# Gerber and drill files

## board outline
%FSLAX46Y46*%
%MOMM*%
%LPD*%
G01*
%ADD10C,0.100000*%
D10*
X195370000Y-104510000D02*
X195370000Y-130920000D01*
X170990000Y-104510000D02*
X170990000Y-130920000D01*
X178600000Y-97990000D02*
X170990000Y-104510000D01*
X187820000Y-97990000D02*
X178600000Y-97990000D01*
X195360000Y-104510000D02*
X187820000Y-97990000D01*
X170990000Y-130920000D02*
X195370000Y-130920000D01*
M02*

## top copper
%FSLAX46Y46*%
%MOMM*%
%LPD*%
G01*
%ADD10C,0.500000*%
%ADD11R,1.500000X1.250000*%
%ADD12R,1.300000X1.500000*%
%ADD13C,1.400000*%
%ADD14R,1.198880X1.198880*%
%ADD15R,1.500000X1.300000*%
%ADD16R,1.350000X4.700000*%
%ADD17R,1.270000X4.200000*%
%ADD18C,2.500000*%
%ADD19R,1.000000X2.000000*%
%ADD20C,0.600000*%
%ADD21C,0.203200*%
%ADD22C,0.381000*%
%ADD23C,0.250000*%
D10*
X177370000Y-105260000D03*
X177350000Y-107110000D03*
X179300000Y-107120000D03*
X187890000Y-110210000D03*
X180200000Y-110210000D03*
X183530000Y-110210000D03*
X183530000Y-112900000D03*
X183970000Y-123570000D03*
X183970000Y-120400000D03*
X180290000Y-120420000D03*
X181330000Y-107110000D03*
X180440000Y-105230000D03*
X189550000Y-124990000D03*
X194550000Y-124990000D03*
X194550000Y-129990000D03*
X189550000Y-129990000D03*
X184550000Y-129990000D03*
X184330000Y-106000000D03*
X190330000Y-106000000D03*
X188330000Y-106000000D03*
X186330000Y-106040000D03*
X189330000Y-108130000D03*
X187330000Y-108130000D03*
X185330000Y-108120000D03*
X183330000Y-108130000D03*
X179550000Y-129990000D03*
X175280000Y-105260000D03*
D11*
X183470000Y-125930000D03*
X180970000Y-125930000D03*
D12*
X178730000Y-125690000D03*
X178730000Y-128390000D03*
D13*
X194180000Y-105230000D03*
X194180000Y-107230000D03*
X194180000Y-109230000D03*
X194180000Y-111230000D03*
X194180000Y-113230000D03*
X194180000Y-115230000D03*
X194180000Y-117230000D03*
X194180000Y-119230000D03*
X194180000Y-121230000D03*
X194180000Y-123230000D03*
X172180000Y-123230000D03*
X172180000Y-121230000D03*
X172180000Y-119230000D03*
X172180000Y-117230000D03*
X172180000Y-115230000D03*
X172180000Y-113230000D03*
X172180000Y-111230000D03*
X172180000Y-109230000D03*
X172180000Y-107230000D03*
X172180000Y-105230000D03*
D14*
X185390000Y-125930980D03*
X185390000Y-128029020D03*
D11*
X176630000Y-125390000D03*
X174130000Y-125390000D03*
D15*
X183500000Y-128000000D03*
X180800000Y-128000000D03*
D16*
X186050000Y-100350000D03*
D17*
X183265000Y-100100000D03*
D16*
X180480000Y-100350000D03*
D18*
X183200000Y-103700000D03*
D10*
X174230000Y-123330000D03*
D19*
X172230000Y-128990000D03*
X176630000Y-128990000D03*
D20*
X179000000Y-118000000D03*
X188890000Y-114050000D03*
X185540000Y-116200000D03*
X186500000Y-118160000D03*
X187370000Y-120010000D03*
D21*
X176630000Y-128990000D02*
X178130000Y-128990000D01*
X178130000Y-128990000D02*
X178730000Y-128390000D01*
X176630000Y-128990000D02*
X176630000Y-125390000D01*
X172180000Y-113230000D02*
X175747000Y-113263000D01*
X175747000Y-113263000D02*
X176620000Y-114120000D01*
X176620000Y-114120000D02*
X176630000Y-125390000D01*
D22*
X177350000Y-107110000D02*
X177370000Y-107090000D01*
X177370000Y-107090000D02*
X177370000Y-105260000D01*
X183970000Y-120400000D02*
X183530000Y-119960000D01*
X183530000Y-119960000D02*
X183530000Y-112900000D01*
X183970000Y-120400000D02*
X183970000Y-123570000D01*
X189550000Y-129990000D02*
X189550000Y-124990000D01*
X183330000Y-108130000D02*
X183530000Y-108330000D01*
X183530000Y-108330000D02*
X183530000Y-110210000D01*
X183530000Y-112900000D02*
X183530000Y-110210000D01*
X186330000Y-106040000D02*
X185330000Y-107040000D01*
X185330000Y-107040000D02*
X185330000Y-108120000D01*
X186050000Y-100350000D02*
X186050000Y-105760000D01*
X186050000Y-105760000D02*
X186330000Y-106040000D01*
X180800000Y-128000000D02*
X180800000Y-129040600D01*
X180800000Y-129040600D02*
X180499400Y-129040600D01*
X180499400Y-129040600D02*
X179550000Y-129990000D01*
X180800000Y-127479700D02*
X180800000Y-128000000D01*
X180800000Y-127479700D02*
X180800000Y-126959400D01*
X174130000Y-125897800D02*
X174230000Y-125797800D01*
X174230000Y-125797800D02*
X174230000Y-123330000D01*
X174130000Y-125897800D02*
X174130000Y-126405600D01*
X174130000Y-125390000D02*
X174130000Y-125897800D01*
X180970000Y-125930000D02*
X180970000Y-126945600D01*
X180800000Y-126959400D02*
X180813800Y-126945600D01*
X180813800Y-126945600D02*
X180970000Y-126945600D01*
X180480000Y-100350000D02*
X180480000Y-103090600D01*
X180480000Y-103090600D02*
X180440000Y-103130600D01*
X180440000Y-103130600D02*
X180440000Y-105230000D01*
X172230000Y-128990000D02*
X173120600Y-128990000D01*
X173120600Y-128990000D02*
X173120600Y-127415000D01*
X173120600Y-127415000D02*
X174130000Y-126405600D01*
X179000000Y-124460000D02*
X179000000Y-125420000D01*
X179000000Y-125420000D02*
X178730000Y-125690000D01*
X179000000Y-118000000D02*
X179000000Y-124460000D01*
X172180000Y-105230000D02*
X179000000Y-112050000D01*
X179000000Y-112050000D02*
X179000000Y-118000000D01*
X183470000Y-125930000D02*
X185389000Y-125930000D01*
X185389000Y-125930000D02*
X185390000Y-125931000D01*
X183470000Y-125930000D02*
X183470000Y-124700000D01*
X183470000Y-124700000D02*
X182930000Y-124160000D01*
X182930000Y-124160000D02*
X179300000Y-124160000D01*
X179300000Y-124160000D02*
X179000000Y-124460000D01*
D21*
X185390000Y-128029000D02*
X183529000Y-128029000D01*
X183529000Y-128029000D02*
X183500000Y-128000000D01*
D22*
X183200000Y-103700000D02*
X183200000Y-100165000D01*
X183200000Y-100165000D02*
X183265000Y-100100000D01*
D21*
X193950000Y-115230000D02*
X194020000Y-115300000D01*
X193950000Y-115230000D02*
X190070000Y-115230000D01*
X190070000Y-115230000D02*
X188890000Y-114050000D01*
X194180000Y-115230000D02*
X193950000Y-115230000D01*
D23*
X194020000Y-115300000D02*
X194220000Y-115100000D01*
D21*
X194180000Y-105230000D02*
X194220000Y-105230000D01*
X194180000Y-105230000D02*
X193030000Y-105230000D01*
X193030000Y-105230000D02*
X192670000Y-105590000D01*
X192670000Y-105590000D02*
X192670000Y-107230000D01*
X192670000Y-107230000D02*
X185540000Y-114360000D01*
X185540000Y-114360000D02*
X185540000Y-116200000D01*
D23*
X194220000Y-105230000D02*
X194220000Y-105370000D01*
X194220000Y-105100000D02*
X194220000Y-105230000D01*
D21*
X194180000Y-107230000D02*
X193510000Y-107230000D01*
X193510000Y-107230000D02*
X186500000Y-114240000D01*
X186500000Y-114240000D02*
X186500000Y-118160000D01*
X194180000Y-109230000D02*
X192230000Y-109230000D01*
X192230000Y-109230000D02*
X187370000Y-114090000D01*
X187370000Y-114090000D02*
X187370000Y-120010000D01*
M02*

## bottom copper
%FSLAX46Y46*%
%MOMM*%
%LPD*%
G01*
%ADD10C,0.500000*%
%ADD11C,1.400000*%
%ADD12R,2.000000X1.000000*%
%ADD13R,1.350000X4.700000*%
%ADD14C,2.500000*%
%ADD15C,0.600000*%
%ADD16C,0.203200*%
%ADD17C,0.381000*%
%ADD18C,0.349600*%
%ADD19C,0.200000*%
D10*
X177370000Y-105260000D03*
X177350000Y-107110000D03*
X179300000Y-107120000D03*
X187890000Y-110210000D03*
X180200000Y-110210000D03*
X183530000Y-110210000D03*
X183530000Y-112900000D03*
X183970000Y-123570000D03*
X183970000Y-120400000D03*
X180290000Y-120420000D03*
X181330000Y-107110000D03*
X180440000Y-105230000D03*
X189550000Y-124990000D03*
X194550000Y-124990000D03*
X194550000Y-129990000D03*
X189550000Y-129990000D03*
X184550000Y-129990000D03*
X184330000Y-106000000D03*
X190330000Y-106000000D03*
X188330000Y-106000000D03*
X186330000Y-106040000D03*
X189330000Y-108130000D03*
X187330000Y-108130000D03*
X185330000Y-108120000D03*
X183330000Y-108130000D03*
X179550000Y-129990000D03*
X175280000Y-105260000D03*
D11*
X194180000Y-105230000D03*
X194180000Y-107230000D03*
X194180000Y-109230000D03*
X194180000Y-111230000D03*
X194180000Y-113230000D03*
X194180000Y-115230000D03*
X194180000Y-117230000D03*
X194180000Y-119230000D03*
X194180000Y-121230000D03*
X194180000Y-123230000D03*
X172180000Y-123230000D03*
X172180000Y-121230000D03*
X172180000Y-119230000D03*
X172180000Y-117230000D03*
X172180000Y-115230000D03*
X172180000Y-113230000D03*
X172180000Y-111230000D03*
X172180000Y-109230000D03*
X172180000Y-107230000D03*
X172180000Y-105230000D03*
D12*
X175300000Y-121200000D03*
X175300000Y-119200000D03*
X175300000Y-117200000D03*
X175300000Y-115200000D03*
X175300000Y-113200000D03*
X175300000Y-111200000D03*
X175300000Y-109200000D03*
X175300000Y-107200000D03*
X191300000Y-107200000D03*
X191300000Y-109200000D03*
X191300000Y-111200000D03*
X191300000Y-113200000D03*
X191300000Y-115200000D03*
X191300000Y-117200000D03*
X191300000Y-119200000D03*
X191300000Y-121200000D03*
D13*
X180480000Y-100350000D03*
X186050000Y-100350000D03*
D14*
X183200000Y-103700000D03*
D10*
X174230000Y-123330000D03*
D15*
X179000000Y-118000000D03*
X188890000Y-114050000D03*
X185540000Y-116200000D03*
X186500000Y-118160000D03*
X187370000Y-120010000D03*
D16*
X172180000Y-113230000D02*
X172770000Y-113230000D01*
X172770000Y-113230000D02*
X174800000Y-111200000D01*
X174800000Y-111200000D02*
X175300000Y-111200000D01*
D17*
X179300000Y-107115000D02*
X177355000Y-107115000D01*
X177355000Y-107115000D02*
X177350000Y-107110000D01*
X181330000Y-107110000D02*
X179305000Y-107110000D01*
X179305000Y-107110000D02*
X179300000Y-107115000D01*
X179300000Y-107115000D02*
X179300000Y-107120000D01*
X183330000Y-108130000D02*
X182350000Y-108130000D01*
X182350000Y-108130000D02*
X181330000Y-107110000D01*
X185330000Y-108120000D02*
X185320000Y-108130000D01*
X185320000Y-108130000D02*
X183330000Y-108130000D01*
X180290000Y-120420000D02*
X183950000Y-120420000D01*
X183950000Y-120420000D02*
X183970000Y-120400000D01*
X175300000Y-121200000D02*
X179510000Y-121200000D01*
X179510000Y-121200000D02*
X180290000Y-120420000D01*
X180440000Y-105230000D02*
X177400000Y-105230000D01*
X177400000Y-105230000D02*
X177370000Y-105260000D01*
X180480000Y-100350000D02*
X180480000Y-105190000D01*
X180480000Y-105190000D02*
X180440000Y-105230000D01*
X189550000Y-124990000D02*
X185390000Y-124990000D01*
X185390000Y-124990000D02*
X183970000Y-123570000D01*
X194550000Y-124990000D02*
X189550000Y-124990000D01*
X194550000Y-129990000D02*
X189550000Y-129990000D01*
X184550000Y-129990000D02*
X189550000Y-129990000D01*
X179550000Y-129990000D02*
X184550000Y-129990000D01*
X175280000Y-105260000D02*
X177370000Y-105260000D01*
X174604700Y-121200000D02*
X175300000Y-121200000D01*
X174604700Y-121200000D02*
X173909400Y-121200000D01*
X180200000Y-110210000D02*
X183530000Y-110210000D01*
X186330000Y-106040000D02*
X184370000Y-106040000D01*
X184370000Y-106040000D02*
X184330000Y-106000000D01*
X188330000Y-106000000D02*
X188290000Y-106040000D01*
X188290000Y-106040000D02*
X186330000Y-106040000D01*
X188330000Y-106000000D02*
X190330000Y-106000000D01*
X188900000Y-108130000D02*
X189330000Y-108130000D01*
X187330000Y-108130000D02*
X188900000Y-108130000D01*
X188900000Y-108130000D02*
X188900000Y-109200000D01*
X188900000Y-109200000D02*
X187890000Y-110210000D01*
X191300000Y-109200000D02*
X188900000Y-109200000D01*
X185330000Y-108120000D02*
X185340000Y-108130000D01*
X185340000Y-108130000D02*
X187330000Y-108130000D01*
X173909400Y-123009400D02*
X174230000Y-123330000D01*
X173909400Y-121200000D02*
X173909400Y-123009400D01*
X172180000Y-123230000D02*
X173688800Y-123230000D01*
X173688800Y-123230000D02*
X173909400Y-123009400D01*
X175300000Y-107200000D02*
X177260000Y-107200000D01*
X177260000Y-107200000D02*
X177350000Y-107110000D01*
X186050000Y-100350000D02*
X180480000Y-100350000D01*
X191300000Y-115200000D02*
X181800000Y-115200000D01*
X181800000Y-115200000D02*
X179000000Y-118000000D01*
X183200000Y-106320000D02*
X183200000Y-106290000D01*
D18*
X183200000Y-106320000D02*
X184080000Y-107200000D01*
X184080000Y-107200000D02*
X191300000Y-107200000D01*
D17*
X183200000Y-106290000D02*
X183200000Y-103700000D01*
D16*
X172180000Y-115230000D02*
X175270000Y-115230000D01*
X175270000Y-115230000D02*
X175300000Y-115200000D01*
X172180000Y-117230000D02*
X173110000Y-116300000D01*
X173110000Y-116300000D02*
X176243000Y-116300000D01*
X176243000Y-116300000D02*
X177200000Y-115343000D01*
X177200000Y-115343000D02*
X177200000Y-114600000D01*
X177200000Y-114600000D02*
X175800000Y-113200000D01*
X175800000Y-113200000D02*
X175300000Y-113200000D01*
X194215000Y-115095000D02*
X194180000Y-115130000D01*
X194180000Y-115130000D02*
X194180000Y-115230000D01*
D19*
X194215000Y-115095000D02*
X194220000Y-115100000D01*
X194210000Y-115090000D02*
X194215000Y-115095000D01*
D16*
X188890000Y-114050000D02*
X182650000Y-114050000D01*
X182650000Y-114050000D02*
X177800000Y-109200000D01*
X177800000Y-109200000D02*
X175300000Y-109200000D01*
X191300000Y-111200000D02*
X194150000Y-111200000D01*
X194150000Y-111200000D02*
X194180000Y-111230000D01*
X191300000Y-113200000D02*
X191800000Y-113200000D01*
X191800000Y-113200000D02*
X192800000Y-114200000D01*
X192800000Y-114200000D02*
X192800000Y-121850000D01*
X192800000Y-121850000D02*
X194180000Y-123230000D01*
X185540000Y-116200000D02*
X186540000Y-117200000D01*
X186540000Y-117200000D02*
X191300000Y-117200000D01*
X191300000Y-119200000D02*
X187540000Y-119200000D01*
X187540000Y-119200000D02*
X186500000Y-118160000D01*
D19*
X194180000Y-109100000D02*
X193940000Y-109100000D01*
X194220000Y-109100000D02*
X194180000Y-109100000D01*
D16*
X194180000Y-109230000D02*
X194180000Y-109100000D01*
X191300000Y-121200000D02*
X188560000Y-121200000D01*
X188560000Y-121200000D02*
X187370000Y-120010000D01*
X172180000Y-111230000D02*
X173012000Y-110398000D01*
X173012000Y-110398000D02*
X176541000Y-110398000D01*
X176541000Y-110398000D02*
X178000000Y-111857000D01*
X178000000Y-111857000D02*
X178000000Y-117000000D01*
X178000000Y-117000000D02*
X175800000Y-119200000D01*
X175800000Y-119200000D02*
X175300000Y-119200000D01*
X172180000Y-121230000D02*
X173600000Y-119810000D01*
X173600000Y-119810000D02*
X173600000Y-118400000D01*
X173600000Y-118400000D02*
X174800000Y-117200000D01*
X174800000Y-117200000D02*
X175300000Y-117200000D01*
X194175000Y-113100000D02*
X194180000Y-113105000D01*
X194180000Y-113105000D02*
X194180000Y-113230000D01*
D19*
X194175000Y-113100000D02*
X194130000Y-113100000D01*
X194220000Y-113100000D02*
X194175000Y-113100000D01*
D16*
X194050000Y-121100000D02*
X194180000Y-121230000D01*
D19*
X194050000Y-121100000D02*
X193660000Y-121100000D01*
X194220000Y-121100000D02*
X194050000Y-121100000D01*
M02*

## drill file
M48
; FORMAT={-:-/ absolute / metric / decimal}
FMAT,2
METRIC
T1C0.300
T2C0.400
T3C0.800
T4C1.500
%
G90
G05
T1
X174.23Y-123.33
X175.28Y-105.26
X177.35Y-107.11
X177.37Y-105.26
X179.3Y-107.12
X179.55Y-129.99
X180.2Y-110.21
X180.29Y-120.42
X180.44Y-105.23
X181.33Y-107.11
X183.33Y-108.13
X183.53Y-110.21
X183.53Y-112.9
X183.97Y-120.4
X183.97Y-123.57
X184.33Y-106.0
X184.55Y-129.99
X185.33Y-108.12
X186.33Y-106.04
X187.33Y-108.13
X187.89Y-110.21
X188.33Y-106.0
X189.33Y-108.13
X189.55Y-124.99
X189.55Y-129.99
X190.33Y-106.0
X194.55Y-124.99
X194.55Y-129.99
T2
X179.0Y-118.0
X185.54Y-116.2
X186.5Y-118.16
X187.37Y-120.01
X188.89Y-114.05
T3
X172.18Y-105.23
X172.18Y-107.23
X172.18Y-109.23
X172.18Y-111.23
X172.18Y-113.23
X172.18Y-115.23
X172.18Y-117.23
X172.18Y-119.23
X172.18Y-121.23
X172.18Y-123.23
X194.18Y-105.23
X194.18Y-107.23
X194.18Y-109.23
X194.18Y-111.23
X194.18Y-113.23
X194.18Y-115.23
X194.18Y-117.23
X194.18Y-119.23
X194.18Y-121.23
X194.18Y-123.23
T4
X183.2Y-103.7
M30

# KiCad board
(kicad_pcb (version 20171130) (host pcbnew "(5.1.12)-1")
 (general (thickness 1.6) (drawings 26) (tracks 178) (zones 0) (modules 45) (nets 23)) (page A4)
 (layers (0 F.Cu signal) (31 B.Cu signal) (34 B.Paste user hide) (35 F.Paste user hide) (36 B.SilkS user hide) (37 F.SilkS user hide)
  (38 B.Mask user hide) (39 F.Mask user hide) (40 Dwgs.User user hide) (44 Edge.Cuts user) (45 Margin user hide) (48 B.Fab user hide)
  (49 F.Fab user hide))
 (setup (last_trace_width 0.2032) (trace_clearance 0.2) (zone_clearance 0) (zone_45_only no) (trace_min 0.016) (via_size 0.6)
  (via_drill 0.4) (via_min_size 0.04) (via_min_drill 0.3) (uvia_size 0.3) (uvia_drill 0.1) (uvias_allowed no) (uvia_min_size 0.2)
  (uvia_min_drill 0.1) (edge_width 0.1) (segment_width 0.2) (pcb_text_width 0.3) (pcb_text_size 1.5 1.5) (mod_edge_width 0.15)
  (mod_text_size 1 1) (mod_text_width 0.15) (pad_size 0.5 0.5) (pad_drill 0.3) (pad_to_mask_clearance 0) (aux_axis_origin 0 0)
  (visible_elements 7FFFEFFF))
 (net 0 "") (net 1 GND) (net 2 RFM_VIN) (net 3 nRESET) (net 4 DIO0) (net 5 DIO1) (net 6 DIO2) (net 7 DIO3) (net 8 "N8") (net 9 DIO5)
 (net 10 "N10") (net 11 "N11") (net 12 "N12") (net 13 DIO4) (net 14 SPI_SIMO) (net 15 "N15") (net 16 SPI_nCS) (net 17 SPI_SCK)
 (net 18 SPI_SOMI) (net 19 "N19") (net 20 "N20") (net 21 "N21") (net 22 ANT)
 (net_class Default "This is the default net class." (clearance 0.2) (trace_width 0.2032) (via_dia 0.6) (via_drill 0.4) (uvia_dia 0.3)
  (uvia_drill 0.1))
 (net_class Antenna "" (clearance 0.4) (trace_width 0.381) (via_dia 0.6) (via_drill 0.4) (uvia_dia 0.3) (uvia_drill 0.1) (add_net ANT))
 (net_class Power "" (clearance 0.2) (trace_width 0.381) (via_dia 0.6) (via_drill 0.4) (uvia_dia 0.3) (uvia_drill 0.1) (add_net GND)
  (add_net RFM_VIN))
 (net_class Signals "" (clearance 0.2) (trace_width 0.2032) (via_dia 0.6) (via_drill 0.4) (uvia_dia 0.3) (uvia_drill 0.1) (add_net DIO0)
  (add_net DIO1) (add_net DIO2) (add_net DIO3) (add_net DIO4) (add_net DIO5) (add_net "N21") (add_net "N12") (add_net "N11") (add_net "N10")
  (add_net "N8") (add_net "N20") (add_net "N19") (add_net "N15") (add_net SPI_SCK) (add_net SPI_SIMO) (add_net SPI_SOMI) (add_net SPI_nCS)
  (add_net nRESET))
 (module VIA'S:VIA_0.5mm (layer F.Cu) (at 177.37 105.26)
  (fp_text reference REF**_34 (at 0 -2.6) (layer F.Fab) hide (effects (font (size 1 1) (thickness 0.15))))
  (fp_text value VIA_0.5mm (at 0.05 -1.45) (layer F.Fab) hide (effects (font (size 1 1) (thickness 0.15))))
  (pad 1 thru_hole circle (at 0 0) (size 0.5 0.5) (drill 0.3) (layers *.Cu) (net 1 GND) (zone_connect 2)))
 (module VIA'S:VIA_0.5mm (layer F.Cu) (at 177.35 107.11)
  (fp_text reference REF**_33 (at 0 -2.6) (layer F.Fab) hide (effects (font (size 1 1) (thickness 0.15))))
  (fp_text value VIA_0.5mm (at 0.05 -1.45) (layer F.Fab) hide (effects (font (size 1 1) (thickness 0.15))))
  (pad 1 thru_hole circle (at 0 0) (size 0.5 0.5) (drill 0.3) (layers *.Cu) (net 1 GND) (zone_connect 2)))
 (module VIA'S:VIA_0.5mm (layer F.Cu) (at 179.3 107.12)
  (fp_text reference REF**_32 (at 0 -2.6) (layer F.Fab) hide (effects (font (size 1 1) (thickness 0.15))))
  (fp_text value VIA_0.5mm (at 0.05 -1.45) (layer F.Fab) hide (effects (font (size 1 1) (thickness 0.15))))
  (pad 1 thru_hole circle (at 0 0) (size 0.5 0.5) (drill 0.3) (layers *.Cu) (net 1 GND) (zone_connect 2)))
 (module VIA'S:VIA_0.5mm (layer F.Cu) (at 186.03 105.9)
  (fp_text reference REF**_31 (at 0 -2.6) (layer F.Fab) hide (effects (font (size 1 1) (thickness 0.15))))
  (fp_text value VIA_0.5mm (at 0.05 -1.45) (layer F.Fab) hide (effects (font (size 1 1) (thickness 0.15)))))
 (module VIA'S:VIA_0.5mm (layer F.Cu) (at 187.89 110.29)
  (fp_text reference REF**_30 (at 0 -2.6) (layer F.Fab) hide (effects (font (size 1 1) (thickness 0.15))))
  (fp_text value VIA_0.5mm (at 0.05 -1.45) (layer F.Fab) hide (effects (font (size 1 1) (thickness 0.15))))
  (pad 1 thru_hole circle (at 0 -0.08) (size 0.5 0.5) (drill 0.3) (layers *.Cu) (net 1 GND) (zone_connect 2)))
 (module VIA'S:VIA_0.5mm (layer F.Cu) (at 180.2 110.23)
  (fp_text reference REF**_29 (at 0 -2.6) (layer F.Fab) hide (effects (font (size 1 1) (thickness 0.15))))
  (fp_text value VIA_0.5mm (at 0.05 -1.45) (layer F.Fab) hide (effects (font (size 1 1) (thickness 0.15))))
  (pad 1 thru_hole circle (at 0 -0.02) (size 0.5 0.5) (drill 0.3) (layers *.Cu) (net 1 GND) (zone_connect 2)))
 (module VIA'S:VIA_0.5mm (layer F.Cu) (at 183.53 110.21)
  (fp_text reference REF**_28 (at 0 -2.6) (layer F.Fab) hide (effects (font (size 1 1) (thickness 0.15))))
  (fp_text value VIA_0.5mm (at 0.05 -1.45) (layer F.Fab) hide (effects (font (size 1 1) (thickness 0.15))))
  (pad 1 thru_hole circle (at 0 0) (size 0.5 0.5) (drill 0.3) (layers *.Cu) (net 1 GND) (zone_connect 2)))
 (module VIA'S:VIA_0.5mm (layer F.Cu) (at 183.54 112.9)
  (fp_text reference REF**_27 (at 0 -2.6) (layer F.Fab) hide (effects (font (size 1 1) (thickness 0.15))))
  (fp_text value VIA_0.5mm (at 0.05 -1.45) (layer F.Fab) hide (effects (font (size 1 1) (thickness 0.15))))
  (pad 1 thru_hole circle (at -0.01 0) (size 0.5 0.5) (drill 0.3) (layers *.Cu) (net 1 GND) (zone_connect 2)))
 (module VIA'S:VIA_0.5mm (layer F.Cu) (at 183.97 123.57)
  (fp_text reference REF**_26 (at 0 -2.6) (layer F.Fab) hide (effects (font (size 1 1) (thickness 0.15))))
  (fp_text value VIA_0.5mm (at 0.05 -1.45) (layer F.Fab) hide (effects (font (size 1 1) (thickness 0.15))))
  (pad 1 thru_hole circle (at 0 0) (size 0.5 0.5) (drill 0.3) (layers *.Cu) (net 1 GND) (zone_connect 2)))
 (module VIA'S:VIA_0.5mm (layer F.Cu) (at 183.97 120.4)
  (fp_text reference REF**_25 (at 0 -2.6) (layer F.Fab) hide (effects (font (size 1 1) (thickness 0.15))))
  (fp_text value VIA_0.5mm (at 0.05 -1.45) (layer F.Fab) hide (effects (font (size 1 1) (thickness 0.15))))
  (pad 1 thru_hole circle (at 0 0) (size 0.5 0.5) (drill 0.3) (layers *.Cu) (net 1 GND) (zone_connect 2)))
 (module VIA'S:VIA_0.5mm (layer F.Cu) (at 180.29 120.42)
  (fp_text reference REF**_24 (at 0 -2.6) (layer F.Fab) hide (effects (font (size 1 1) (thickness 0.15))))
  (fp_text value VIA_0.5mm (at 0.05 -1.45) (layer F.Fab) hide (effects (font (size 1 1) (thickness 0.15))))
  (pad 1 thru_hole circle (at 0 0) (size 0.5 0.5) (drill 0.3) (layers *.Cu) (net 1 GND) (zone_connect 2)))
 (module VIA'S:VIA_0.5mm (layer F.Cu) (at 181.33 107.11)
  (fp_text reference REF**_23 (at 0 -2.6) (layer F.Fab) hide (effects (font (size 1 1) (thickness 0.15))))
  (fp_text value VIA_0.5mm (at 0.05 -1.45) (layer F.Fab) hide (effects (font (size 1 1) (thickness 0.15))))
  (pad 1 thru_hole circle (at 0 0) (size 0.5 0.5) (drill 0.3) (layers *.Cu) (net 1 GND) (zone_connect 2)))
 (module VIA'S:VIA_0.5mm (layer F.Cu) (at 180.44 105.23)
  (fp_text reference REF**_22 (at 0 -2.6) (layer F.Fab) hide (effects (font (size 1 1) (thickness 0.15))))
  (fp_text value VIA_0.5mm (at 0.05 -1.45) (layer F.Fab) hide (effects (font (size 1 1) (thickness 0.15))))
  (pad 1 thru_hole circle (at 0 0) (size 0.5 0.5) (drill 0.3) (layers *.Cu) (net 1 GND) (zone_connect 2)))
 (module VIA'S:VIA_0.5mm (layer F.Cu) (at 189.55 124.99)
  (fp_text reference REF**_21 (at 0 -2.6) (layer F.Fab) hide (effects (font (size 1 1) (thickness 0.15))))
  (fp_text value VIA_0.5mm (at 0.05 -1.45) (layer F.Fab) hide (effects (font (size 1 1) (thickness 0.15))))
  (pad 1 thru_hole circle (at 0 0) (size 0.5 0.5) (drill 0.3) (layers *.Cu) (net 1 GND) (zone_connect 2)))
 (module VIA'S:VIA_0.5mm (layer F.Cu) (at 194.55 124.99)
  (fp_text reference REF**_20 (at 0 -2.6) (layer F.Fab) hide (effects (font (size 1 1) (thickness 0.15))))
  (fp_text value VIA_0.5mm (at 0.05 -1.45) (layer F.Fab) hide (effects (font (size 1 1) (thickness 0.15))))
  (pad 1 thru_hole circle (at 0 0) (size 0.5 0.5) (drill 0.3) (layers *.Cu) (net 1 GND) (zone_connect 2)))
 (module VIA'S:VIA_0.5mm (layer F.Cu) (at 194.55 129.99)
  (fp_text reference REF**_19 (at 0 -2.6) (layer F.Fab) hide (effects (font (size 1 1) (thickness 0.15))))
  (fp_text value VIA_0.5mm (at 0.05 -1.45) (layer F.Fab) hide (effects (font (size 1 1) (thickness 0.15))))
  (pad 1 thru_hole circle (at 0 0) (size 0.5 0.5) (drill 0.3) (layers *.Cu) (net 1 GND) (zone_connect 2)))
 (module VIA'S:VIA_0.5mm (layer F.Cu) (at 189.55 129.99)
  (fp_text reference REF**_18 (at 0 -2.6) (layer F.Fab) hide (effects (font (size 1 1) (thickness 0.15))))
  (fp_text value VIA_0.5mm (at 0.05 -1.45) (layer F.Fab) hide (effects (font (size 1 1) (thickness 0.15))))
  (pad 1 thru_hole circle (at 0 0) (size 0.5 0.5) (drill 0.3) (layers *.Cu) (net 1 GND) (zone_connect 2)))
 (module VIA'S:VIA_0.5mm (layer F.Cu) (at 184.55 129.99)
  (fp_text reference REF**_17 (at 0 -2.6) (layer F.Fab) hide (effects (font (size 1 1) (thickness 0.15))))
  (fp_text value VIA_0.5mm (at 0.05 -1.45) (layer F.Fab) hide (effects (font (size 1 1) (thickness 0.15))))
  (pad 1 thru_hole circle (at 0 0) (size 0.5 0.5) (drill 0.3) (layers *.Cu) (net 1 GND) (zone_connect 2)))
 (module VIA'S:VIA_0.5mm (layer F.Cu) (at 184.33 106.67)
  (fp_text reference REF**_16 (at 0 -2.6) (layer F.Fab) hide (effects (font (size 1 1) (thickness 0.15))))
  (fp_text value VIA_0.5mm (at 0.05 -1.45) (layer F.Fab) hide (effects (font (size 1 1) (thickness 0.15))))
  (pad 1 thru_hole circle (at 0 -0.67) (size 0.5 0.5) (drill 0.3) (layers *.Cu) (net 1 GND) (zone_connect 2)))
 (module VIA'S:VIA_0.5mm (layer F.Cu) (at 189.33 106.67)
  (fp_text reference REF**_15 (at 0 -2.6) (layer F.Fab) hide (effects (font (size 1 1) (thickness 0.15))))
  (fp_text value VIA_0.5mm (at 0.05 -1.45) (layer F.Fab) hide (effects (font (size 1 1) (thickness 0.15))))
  (pad 1 thru_hole circle (at 1 -0.67) (size 0.5 0.5) (drill 0.3) (layers *.Cu) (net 1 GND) (zone_connect 2)))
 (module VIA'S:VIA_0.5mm (layer F.Cu) (at 188.33 106.67)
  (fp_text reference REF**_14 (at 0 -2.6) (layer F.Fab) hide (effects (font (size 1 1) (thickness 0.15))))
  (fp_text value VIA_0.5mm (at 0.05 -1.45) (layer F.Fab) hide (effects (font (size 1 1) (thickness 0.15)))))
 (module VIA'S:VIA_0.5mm (layer F.Cu) (at 187.33 106.67)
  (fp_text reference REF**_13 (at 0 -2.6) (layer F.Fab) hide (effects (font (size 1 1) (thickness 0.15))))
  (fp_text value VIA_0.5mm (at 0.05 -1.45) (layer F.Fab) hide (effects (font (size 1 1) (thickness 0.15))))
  (pad 1 thru_hole circle (at 1 -0.67) (size 0.5 0.5) (drill 0.3) (layers *.Cu) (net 1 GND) (zone_connect 2)))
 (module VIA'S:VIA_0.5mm (layer F.Cu) (at 186.33 106.67)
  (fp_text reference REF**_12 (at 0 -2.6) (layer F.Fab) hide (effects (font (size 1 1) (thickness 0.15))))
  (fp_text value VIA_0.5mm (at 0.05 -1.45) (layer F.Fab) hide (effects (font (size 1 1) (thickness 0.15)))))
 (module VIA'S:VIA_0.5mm (layer F.Cu) (at 186.05 106.71)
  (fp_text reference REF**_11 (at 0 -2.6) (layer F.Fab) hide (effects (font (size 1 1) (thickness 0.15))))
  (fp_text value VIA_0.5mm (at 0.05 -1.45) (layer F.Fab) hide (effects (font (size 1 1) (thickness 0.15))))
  (pad 1 thru_hole circle (at 0.28 -0.67) (size 0.5 0.5) (drill 0.3) (layers *.Cu) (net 1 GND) (zone_connect 2)))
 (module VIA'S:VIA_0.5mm (layer F.Cu) (at 189.03 108.13)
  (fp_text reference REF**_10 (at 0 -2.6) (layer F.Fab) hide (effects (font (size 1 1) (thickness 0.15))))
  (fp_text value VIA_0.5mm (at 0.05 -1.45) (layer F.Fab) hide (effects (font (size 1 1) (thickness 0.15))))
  (pad 1 thru_hole circle (at 0.3 0) (size 0.5 0.5) (drill 0.3) (layers *.Cu) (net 1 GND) (zone_connect 2)))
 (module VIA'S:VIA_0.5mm (layer F.Cu) (at 188.03 108.13)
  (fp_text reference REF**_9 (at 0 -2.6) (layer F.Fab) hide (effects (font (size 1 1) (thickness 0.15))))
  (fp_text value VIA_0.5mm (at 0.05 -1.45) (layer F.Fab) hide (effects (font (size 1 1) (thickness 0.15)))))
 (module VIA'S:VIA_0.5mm (layer F.Cu) (at 187.03 108.13)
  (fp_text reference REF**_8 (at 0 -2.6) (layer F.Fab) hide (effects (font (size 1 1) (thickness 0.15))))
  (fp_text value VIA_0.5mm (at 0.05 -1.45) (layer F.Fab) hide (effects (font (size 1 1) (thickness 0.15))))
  (pad 1 thru_hole circle (at 0.3 0) (size 0.5 0.5) (drill 0.3) (layers *.Cu) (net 1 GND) (zone_connect 2)))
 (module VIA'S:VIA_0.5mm (layer F.Cu) (at 186.03 108.13)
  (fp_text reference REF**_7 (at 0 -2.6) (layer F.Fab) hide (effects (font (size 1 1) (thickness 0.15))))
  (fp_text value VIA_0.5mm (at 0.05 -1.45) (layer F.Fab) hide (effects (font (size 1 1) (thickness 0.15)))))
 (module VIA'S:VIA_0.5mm (layer F.Cu) (at 185.54 108.12)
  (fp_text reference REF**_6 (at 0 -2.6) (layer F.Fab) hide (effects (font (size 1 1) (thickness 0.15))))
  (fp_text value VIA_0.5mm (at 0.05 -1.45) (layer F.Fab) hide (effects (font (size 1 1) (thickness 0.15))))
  (pad 1 thru_hole circle (at -0.21 0) (size 0.5 0.5) (drill 0.3) (layers *.Cu) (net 1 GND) (zone_connect 2)))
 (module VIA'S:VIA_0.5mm (layer F.Cu) (at 184.03 108.13)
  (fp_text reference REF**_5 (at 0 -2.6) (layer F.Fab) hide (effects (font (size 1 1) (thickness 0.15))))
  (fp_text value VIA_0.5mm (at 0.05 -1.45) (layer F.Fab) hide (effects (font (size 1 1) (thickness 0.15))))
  (pad 1 thru_hole circle (at -0.7 0) (size 0.5 0.5) (drill 0.3) (layers *.Cu) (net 1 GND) (zone_connect 2)))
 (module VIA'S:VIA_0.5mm (layer F.Cu) (at 179.55 129.99)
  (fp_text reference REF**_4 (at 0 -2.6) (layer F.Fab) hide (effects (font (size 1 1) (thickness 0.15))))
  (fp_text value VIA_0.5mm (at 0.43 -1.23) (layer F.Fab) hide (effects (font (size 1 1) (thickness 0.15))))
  (pad 1 thru_hole circle (at 0 0) (size 0.5 0.5) (drill 0.3) (layers *.Cu) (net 1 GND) (zone_connect 2)))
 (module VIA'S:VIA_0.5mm (layer F.Cu) (at 175.28 105.26)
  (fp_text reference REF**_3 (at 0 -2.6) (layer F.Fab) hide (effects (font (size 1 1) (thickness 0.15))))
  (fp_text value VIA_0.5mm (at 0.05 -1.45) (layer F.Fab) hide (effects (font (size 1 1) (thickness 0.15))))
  (pad 1 thru_hole circle (at 0 0) (size 0.5 0.5) (drill 0.3) (layers *.Cu) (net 1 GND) (zone_connect 2)))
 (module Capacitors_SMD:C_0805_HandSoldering (layer F.Cu) (at 182.22 125.93 180)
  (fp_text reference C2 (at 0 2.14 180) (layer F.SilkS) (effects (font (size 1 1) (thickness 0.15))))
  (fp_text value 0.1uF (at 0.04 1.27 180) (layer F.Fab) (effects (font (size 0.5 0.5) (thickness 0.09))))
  (pad 1 smd rect (at -1.25 0 180) (size 1.5 1.25) (layers F.Cu F.Paste F.Mask) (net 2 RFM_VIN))
  (pad 2 smd rect (at 1.25 0 180) (size 1.5 1.25) (layers F.Cu F.Paste F.Mask) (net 1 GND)))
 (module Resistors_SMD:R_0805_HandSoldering (layer F.Cu) (at 178.73 127.04 270)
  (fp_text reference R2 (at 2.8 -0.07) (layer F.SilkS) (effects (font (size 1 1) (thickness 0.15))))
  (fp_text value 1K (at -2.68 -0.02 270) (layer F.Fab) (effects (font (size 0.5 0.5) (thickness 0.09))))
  (pad 1 smd rect (at -1.35 0 270) (size 1.5 1.3) (layers F.Cu F.Paste F.Mask) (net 2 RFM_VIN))
  (pad 2 smd rect (at 1.35 0 270) (size 1.5 1.3) (layers F.Cu F.Paste F.Mask) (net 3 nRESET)))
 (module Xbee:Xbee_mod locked (layer F.Cu) (at 172.18 105.23)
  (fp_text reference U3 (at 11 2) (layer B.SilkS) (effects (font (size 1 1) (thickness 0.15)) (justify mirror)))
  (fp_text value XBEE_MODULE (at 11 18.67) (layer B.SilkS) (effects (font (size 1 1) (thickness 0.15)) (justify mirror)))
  (pad 20 thru_hole circle (at 22 0) (size 1.4 1.4) (drill 0.8) (layers *.Cu *.Mask) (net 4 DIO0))
  (pad 19 thru_hole circle (at 22 2) (size 1.4 1.4) (drill 0.8) (layers *.Cu *.Mask) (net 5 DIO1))
  (pad 18 thru_hole circle (at 22 4) (size 1.4 1.4) (drill 0.8) (layers *.Cu *.Mask) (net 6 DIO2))
  (pad 17 thru_hole circle (at 22 6) (size 1.4 1.4) (drill 0.8) (layers *.Cu *.Mask) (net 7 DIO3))
  (pad 16 thru_hole circle (at 22 8) (size 1.4 1.4) (drill 0.8) (layers *.Cu *.Mask) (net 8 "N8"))
  (pad 15 thru_hole circle (at 22 10) (size 1.4 1.4) (drill 0.8) (layers *.Cu *.Mask) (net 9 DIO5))
  (pad 14 thru_hole circle (at 22 12) (size 1.4 1.4) (drill 0.8) (layers *.Cu *.Mask) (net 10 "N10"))
  (pad 13 thru_hole circle (at 22 14) (size 1.4 1.4) (drill 0.8) (layers *.Cu *.Mask) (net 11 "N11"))
  (pad 12 thru_hole circle (at 22 16) (size 1.4 1.4) (drill 0.8) (layers *.Cu *.Mask) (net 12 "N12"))
  (pad 11 thru_hole circle (at 22 18) (size 1.4 1.4) (drill 0.8) (layers *.Cu *.Mask) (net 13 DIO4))
  (pad 10 thru_hole circle (at 0 18) (size 1.4 1.4) (drill 0.8) (layers *.Cu *.Mask) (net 1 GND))
  (pad 9 thru_hole circle (at 0 16) (size 1.4 1.4) (drill 0.8) (layers *.Cu *.Mask) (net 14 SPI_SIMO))
  (pad 8 thru_hole circle (at 0 14) (size 1.4 1.4) (drill 0.8) (layers *.Cu *.Mask) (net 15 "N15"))
  (pad 7 thru_hole circle (at 0 12) (size 1.4 1.4) (drill 0.8) (layers *.Cu *.Mask) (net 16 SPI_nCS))
  (pad 6 thru_hole circle (at 0 10) (size 1.4 1.4) (drill 0.8) (layers *.Cu *.Mask) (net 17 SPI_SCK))
  (pad 5 thru_hole circle (at 0 8) (size 1.4 1.4) (drill 0.8) (layers *.Cu *.Mask) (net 3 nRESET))
  (pad 4 thru_hole circle (at 0 6) (size 1.4 1.4) (drill 0.8) (layers *.Cu *.Mask) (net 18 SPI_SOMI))
  (pad 3 thru_hole circle (at 0 4) (size 1.4 1.4) (drill 0.8) (layers *.Cu *.Mask) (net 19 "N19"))
  (pad 2 thru_hole circle (at 0 2) (size 1.4 1.4) (drill 0.8) (layers *.Cu *.Mask) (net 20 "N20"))
  (pad 1 thru_hole circle (at 0 0) (size 1.4 1.4) (drill 0.8) (layers *.Cu *.Mask) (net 2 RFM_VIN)))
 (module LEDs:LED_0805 (layer F.Cu) (at 185.39 126.98 90)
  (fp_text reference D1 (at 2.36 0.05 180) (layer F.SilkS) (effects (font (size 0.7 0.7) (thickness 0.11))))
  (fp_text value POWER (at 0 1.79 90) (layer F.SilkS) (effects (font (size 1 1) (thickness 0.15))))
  (pad 2 smd rect (at 1.04902 0 270) (size 1.19888 1.19888) (layers F.Cu F.Paste F.Mask) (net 2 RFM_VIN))
  (pad 1 smd rect (at -1.04902 0 270) (size 1.19888 1.19888) (layers F.Cu F.Paste F.Mask) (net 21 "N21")))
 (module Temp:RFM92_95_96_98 (layer B.Cu) (at 175.3 121.2)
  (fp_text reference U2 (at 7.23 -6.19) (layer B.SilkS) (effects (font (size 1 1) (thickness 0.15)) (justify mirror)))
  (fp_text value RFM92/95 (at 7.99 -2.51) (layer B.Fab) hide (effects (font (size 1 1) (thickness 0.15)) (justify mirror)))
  (pad 1 smd rect (at 0 0) (size 2 1) (layers B.Cu B.Paste B.Mask) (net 1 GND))
  (pad 2 smd rect (at 0 -2) (size 2 1) (layers B.Cu B.Paste B.Mask) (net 18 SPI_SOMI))
  (pad 3 smd rect (at 0 -4) (size 2 1) (layers B.Cu B.Paste B.Mask) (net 14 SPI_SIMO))
  (pad 4 smd rect (at 0 -6) (size 2 1) (layers B.Cu B.Paste B.Mask) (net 17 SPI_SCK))
  (pad 5 smd rect (at 0 -8) (size 2 1) (layers B.Cu B.Paste B.Mask) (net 16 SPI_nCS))
  (pad 6 smd rect (at 0 -10) (size 2 1) (layers B.Cu B.Paste B.Mask) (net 3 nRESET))
  (pad 7 smd rect (at 0 -12) (size 2 1) (layers B.Cu B.Paste B.Mask) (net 9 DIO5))
  (pad 8 smd rect (at 0 -14) (size 2 1) (layers B.Cu B.Paste B.Mask) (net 1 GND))
  (pad 9 smd rect (at 16 -14) (size 2 1) (layers B.Cu B.Paste B.Mask) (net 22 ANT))
  (pad 10 smd rect (at 16 -12) (size 2 1) (layers B.Cu B.Paste B.Mask) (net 1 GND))
  (pad 11 smd rect (at 16 -10) (size 2 1) (layers B.Cu B.Paste B.Mask) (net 7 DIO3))
  (pad 12 smd rect (at 16 -8) (size 2 1) (layers B.Cu B.Paste B.Mask) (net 13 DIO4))
  (pad 13 smd rect (at 16 -6) (size 2 1) (layers B.Cu B.Paste B.Mask) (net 2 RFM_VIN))
  (pad 14 smd rect (at 16 -4) (size 2 1) (layers B.Cu B.Paste B.Mask) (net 4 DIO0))
  (pad 15 smd rect (at 16 -2) (size 2 1) (layers B.Cu B.Paste B.Mask) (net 5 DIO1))
  (pad 16 smd rect (at 16 0) (size 2 1) (layers B.Cu B.Paste B.Mask) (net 6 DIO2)))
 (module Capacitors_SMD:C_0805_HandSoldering (layer F.Cu) (at 175.38 125.39 180)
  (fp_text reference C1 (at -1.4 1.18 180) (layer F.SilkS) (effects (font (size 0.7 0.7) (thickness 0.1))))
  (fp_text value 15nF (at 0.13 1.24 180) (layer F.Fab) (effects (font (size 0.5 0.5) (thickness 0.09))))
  (pad 1 smd rect (at -1.25 0 180) (size 1.5 1.25) (layers F.Cu F.Paste F.Mask) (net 3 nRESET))
  (pad 2 smd rect (at 1.25 0 180) (size 1.5 1.25) (layers F.Cu F.Paste F.Mask) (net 1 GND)))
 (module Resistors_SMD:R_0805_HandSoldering (layer F.Cu) (at 182.15 128 180)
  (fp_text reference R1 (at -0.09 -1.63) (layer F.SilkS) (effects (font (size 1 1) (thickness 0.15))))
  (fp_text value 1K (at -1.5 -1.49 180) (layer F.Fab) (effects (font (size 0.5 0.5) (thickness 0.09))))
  (pad 1 smd rect (at -1.35 0 180) (size 1.5 1.3) (layers F.Cu F.Paste F.Mask) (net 21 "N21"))
  (pad 2 smd rect (at 1.35 0 180) (size 1.5 1.3) (layers F.Cu F.Paste F.Mask) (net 1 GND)))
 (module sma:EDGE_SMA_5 (layer F.Cu) (at 186.05 100.35 270)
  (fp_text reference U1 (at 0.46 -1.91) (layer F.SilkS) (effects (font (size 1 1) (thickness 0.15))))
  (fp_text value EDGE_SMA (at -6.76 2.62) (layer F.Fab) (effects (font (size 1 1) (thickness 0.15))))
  (pad 5 smd rect (at 0 5.57 270) (size 4.7 1.35) (layers B.Cu F.Paste F.Mask) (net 1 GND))
  (pad 3 smd rect (at 0 0 270) (size 4.7 1.35) (layers B.Cu F.Paste F.Mask) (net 1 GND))
  (pad 2 smd rect (at 0 0 270) (size 4.7 1.35) (layers F.Cu F.Paste F.Mask) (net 1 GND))
  (pad 1 smd rect (at -0.25 2.785 270) (size 4.2 1.27) (layers F.Cu F.Paste F.Mask) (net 22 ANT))
  (pad 4 smd rect (at 0 5.57 270) (size 4.7 1.35) (layers F.Cu F.Paste F.Mask) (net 1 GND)))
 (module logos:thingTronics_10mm (layer F.Cu) (at 182.23 117.37)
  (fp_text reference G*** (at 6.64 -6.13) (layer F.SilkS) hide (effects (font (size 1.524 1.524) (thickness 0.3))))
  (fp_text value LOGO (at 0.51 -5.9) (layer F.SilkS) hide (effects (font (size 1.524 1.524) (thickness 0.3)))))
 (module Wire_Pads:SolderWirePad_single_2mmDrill (layer F.Cu) (at 183.2 103.7)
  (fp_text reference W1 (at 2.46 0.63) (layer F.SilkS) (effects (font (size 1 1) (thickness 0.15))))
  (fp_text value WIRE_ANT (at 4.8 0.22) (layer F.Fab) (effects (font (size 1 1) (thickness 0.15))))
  (pad 1 thru_hole circle (at 0 0) (size 2.5 2.5) (drill 1.5) (layers *.Cu F.Mask) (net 22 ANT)))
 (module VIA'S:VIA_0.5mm (layer F.Cu) (at 174.23 123.33)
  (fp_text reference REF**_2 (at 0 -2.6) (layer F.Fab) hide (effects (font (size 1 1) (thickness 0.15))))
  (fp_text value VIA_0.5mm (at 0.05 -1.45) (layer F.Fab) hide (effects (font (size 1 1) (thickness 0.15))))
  (pad 1 thru_hole circle (at 0 0) (size 0.5 0.5) (drill 0.3) (layers *.Cu) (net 1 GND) (zone_connect 2)))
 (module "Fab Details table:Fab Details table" (layer F.Cu) (at 127.11 93.44)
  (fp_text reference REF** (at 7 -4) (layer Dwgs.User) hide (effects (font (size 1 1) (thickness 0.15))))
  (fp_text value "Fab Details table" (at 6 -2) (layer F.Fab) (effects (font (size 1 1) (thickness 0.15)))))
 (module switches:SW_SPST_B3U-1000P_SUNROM (layer F.Cu) (at 174.43 128.99)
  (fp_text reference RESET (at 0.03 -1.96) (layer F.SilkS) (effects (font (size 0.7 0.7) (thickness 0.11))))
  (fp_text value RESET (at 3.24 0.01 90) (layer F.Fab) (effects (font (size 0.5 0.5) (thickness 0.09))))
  (pad 1 smd rect (at -2.2 0) (size 1 2) (layers F.Cu F.Paste F.Mask) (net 1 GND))
  (pad 2 smd rect (at 2.2 0) (size 1 2) (layers F.Cu F.Paste F.Mask) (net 3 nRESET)))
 (gr_line (start 195.37 104.51) (end 195.37 130.92) (layer Edge.Cuts) (width 0.1))
 (gr_line (start 170.99 104.51) (end 170.99 130.92) (layer Edge.Cuts) (width 0.1))
 (gr_line (start 178.6 97.99) (end 170.99 104.51) (layer Edge.Cuts) (width 0.1))
 (gr_line (start 187.82 97.99) (end 178.6 97.99) (layer Edge.Cuts) (width 0.1))
 (gr_line (start 195.36 104.51) (end 187.82 97.99) (layer Edge.Cuts) (width 0.1))
 (gr_line (start 170.99 130.92) (end 195.37 130.92) (layer Edge.Cuts) (width 0.1))
 (segment (start 172.18 113.23) (end 172.77 113.23) (width 0.2032) (layer B.Cu) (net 3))
 (segment (start 172.77 113.23) (end 174.8 111.2) (width 0.2032) (layer B.Cu) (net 3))
 (segment (start 174.8 111.2) (end 175.3 111.2) (width 0.2032) (layer B.Cu) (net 3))
 (segment (start 176.63 128.99) (end 178.13 128.99) (width 0.2032) (layer F.Cu) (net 3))
 (segment (start 178.13 128.99) (end 178.73 128.39) (width 0.2032) (layer F.Cu) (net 3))
 (segment (start 176.63 128.99) (end 176.63 125.39) (width 0.2032) (layer F.Cu) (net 3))
 (segment (start 172.18 113.23) (end 175.747 113.263) (width 0.2032) (layer F.Cu) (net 3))
 (segment (start 175.747 113.263) (end 176.62 114.12) (width 0.2032) (layer F.Cu) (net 3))
 (segment (start 176.62 114.12) (end 176.63 125.39) (width 0.2032) (layer F.Cu) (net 3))
 (segment (start 177.35 107.11) (end 177.37 107.09) (width 0.381) (layer F.Cu) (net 1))
 (segment (start 177.37 107.09) (end 177.37 105.26) (width 0.381) (layer F.Cu) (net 1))
 (segment (start 179.3 107.115) (end 177.355 107.115) (width 0.381) (layer B.Cu) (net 1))
 (segment (start 177.355 107.115) (end 177.35 107.11) (width 0.381) (layer B.Cu) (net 1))
 (segment (start 181.33 107.11) (end 179.305 107.11) (width 0.381) (layer B.Cu) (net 1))
 (segment (start 179.305 107.11) (end 179.3 107.115) (width 0.381) (layer B.Cu) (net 1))
 (segment (start 179.3 107.115) (end 179.3 107.12) (width 0.381) (layer B.Cu) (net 1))
 (segment (start 183.33 108.13) (end 182.35 108.13) (width 0.381) (layer B.Cu) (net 1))
 (segment (start 182.35 108.13) (end 181.33 107.11) (width 0.381) (layer B.Cu) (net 1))
 (segment (start 185.33 108.12) (end 185.32 108.13) (width 0.381) (layer B.Cu) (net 1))
 (segment (start 185.32 108.13) (end 183.33 108.13) (width 0.381) (layer B.Cu) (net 1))
 (segment (start 183.97 120.4) (end 183.53 119.96) (width 0.381) (layer F.Cu) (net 1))
 (segment (start 183.53 119.96) (end 183.53 112.9) (width 0.381) (layer F.Cu) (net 1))
 (segment (start 183.97 120.4) (end 183.97 123.57) (width 0.381) (layer F.Cu) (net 1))
 (segment (start 180.29 120.42) (end 183.95 120.42) (width 0.381) (layer B.Cu) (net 1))
 (segment (start 183.95 120.42) (end 183.97 120.4) (width 0.381) (layer B.Cu) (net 1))
 (segment (start 175.3 121.2) (end 179.51 121.2) (width 0.381) (layer B.Cu) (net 1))
 (segment (start 179.51 121.2) (end 180.29 120.42) (width 0.381) (layer B.Cu) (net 1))
 (segment (start 180.44 105.23) (end 177.4 105.23) (width 0.381) (layer B.Cu) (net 1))
 (segment (start 177.4 105.23) (end 177.37 105.26) (width 0.381) (layer B.Cu) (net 1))
 (segment (start 180.48 100.35) (end 180.48 105.19) (width 0.381) (layer B.Cu) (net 1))
 (segment (start 180.48 105.19) (end 180.44 105.23) (width 0.381) (layer B.Cu) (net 1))
 (segment (start 189.55 124.99) (end 185.39 124.99) (width 0.381) (layer B.Cu) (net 1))
 (segment (start 185.39 124.99) (end 183.97 123.57) (width 0.381) (layer B.Cu) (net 1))
 (segment (start 194.55 124.99) (end 189.55 124.99) (width 0.381) (layer B.Cu) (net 1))
 (segment (start 194.55 129.99) (end 189.55 129.99) (width 0.381) (layer B.Cu) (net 1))
 (segment (start 189.55 129.99) (end 189.55 124.99) (width 0.381) (layer F.Cu) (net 1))
 (segment (start 184.55 129.99) (end 189.55 129.99) (width 0.381) (layer B.Cu) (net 1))
 (segment (start 179.55 129.99) (end 184.55 129.99) (width 0.381) (layer B.Cu) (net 1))
 (segment (start 175.28 105.26) (end 177.37 105.26) (width 0.381) (layer B.Cu) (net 1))
 (segment (start 174.6047 121.2) (end 175.3 121.2) (width 0.381) (layer B.Cu) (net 1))
 (segment (start 174.6047 121.2) (end 173.9094 121.2) (width 0.381) (layer B.Cu) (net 1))
 (segment (start 183.33 108.13) (end 183.53 108.33) (width 0.381) (layer F.Cu) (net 1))
 (segment (start 183.53 108.33) (end 183.53 110.21) (width 0.381) (layer F.Cu) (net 1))
 (segment (start 180.2 110.21) (end 183.53 110.21) (width 0.381) (layer B.Cu) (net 1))
 (segment (start 183.53 112.9) (end 183.53 110.21) (width 0.381) (layer F.Cu) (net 1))
 (segment (start 186.33 106.04) (end 185.33 107.04) (width 0.381) (layer F.Cu) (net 1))
 (segment (start 185.33 107.04) (end 185.33 108.12) (width 0.381) (layer F.Cu) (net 1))
 (segment (start 186.05 100.35) (end 186.05 105.76) (width 0.381) (layer F.Cu) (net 1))
 (segment (start 186.05 105.76) (end 186.33 106.04) (width 0.381) (layer F.Cu) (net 1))
 (segment (start 186.33 106.04) (end 184.37 106.04) (width 0.381) (layer B.Cu) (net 1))
 (segment (start 184.37 106.04) (end 184.33 106) (width 0.381) (layer B.Cu) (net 1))
 (segment (start 188.33 106) (end 188.29 106.04) (width 0.381) (layer B.Cu) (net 1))
 (segment (start 188.29 106.04) (end 186.33 106.04) (width 0.381) (layer B.Cu) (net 1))
 (segment (start 188.33 106) (end 190.33 106) (width 0.381) (layer B.Cu) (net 1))
 (segment (start 188.9 108.13) (end 189.33 108.13) (width 0.381) (layer B.Cu) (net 1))
 (segment (start 187.33 108.13) (end 188.9 108.13) (width 0.381) (layer B.Cu) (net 1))
 (segment (start 188.9 108.13) (end 188.9 109.2) (width 0.381) (layer B.Cu) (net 1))
 (segment (start 188.9 109.2) (end 187.89 110.21) (width 0.381) (layer B.Cu) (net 1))
 (segment (start 191.3 109.2) (end 188.9 109.2) (width 0.381) (layer B.Cu) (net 1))
 (segment (start 185.33 108.12) (end 185.34 108.13) (width 0.381) (layer B.Cu) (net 1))
 (segment (start 185.34 108.13) (end 187.33 108.13) (width 0.381) (layer B.Cu) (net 1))
 (segment (start 180.8 128) (end 180.8 129.0406) (width 0.381) (layer F.Cu) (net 1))
 (segment (start 180.8 129.0406) (end 180.4994 129.0406) (width 0.381) (layer F.Cu) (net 1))
 (segment (start 180.4994 129.0406) (end 179.55 129.99) (width 0.381) (layer F.Cu) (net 1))
 (segment (start 180.8 127.4797) (end 180.8 128) (width 0.381) (layer F.Cu) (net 1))
 (segment (start 180.8 127.4797) (end 180.8 126.9594) (width 0.381) (layer F.Cu) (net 1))
 (segment (start 174.13 125.8978) (end 174.23 125.7978) (width 0.381) (layer F.Cu) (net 1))
 (segment (start 174.23 125.7978) (end 174.23 123.33) (width 0.381) (layer F.Cu) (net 1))
 (segment (start 174.13 125.8978) (end 174.13 126.4056) (width 0.381) (layer F.Cu) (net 1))
 (segment (start 174.13 125.39) (end 174.13 125.8978) (width 0.381) (layer F.Cu) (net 1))
 (segment (start 180.97 125.93) (end 180.97 126.9456) (width 0.381) (layer F.Cu) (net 1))
 (segment (start 180.8 126.9594) (end 180.8138 126.9456) (width 0.381) (layer F.Cu) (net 1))
 (segment (start 180.8138 126.9456) (end 180.97 126.9456) (width 0.381) (layer F.Cu) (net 1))
 (segment (start 173.9094 123.0094) (end 174.23 123.33) (width 0.381) (layer B.Cu) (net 1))
 (segment (start 173.9094 121.2) (end 173.9094 123.0094) (width 0.381) (layer B.Cu) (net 1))
 (segment (start 172.18 123.23) (end 173.6888 123.23) (width 0.381) (layer B.Cu) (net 1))
 (segment (start 173.6888 123.23) (end 173.9094 123.0094) (width 0.381) (layer B.Cu) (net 1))
 (segment (start 175.3 107.2) (end 177.26 107.2) (width 0.381) (layer B.Cu) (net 1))
 (segment (start 177.26 107.2) (end 177.35 107.11) (width 0.381) (layer B.Cu) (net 1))
 (segment (start 186.05 100.35) (end 180.48 100.35) (width 0.381) (layer B.Cu) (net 1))
 (segment (start 180.48 100.35) (end 180.48 103.0906) (width 0.381) (layer F.Cu) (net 1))
 (segment (start 180.48 103.0906) (end 180.44 103.1306) (width 0.381) (layer F.Cu) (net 1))
 (segment (start 180.44 103.1306) (end 180.44 105.23) (width 0.381) (layer F.Cu) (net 1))
 (segment (start 172.23 128.99) (end 173.1206 128.99) (width 0.381) (layer F.Cu) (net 1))
 (segment (start 173.1206 128.99) (end 173.1206 127.415) (width 0.381) (layer F.Cu) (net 1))
 (segment (start 173.1206 127.415) (end 174.13 126.4056) (width 0.381) (layer F.Cu) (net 1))
 (segment (start 179 124.46) (end 179 125.42) (width 0.381) (layer F.Cu) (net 2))
 (segment (start 179 125.42) (end 178.73 125.69) (width 0.381) (layer F.Cu) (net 2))
 (segment (start 179 118) (end 179 124.46) (width 0.381) (layer F.Cu) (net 2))
 (segment (start 172.18 105.23) (end 179 112.05) (width 0.381) (layer F.Cu) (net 2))
 (segment (start 179 112.05) (end 179 118) (width 0.381) (layer F.Cu) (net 2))
 (segment (start 191.3 115.2) (end 181.8 115.2) (width 0.381) (layer B.Cu) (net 2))
 (segment (start 181.8 115.2) (end 179 118) (width 0.381) (layer B.Cu) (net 2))
 (segment (start 183.47 125.93) (end 185.389 125.93) (width 0.381) (layer F.Cu) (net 2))
 (segment (start 185.389 125.93) (end 185.39 125.931) (width 0.381) (layer F.Cu) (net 2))
 (segment (start 183.47 125.93) (end 183.47 124.7) (width 0.381) (layer F.Cu) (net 2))
 (segment (start 183.47 124.7) (end 182.93 124.16) (width 0.381) (layer F.Cu) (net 2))
 (segment (start 182.93 124.16) (end 179.3 124.16) (width 0.381) (layer F.Cu) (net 2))
 (segment (start 179.3 124.16) (end 179 124.46) (width 0.381) (layer F.Cu) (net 2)) (via (at 179 118) (size 0.6) (layers F.Cu B.Cu) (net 2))
 (segment (start 185.39 128.029) (end 183.529 128.029) (width 0.2032) (layer F.Cu) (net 21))
 (segment (start 183.529 128.029) (end 183.5 128) (width 0.2032) (layer F.Cu) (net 21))
 (segment (start 183.2 106.32) (end 183.2 106.29) (width 0.381) (layer B.Cu) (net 22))
 (segment (start 183.2 106.32) (end 184.08 107.2) (width 0.3496) (layer B.Cu) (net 22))
 (segment (start 184.08 107.2) (end 191.3 107.2) (width 0.3496) (layer B.Cu) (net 22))
 (segment (start 183.2 106.29) (end 183.2 103.7) (width 0.381) (layer B.Cu) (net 22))
 (segment (start 183.2 103.7) (end 183.2 100.165) (width 0.381) (layer F.Cu) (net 22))
 (segment (start 183.2 100.165) (end 183.265 100.1) (width 0.381) (layer F.Cu) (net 22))
 (segment (start 172.18 115.23) (end 175.27 115.23) (width 0.2032) (layer B.Cu) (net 17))
 (segment (start 175.27 115.23) (end 175.3 115.2) (width 0.2032) (layer B.Cu) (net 17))
 (segment (start 172.18 117.23) (end 173.11 116.3) (width 0.2032) (layer B.Cu) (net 16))
 (segment (start 173.11 116.3) (end 176.243 116.3) (width 0.2032) (layer B.Cu) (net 16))
 (segment (start 176.243 116.3) (end 177.2 115.343) (width 0.2032) (layer B.Cu) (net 16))
 (segment (start 177.2 115.343) (end 177.2 114.6) (width 0.2032) (layer B.Cu) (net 16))
 (segment (start 177.2 114.6) (end 175.8 113.2) (width 0.2032) (layer B.Cu) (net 16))
 (segment (start 175.8 113.2) (end 175.3 113.2) (width 0.2032) (layer B.Cu) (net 16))
 (segment (start 194.215 115.095) (end 194.18 115.13) (width 0.2032) (layer B.Cu) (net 9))
 (segment (start 194.18 115.13) (end 194.18 115.23) (width 0.2032) (layer B.Cu) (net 9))
 (segment (start 194.215 115.095) (end 194.22 115.1) (width 0.2) (layer B.Cu) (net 9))
 (segment (start 194.21 115.09) (end 194.215 115.095) (width 0.2) (layer B.Cu) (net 9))
 (segment (start 193.95 115.23) (end 194.02 115.3) (width 0.2032) (layer F.Cu) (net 9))
 (segment (start 193.95 115.23) (end 190.07 115.23) (width 0.2032) (layer F.Cu) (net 9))
 (segment (start 190.07 115.23) (end 188.89 114.05) (width 0.2032) (layer F.Cu) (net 9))
 (segment (start 194.18 115.23) (end 193.95 115.23) (width 0.2032) (layer F.Cu) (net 9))
 (segment (start 194.02 115.3) (end 194.22 115.1) (width 0.25) (layer F.Cu) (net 9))
 (segment (start 188.89 114.05) (end 182.65 114.05) (width 0.2032) (layer B.Cu) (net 9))
 (segment (start 182.65 114.05) (end 177.8 109.2) (width 0.2032) (layer B.Cu) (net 9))
 (segment (start 177.8 109.2) (end 175.3 109.2) (width 0.2032) (layer B.Cu) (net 9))
 (via (at 188.89 114.05) (size 0.6) (layers F.Cu B.Cu) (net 9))
 (segment (start 191.3 111.2) (end 194.15 111.2) (width 0.2032) (layer B.Cu) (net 7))
 (segment (start 194.15 111.2) (end 194.18 111.23) (width 0.2032) (layer B.Cu) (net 7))
 (segment (start 191.3 113.2) (end 191.8 113.2) (width 0.2032) (layer B.Cu) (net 13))
 (segment (start 191.8 113.2) (end 192.8 114.2) (width 0.2032) (layer B.Cu) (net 13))
 (segment (start 192.8 114.2) (end 192.8 121.85) (width 0.2032) (layer B.Cu) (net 13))
 (segment (start 192.8 121.85) (end 194.18 123.23) (width 0.2032) (layer B.Cu) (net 13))
 (segment (start 194.18 105.23) (end 194.22 105.23) (width 0.2032) (layer F.Cu) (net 4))
 (segment (start 194.18 105.23) (end 193.03 105.23) (width 0.2032) (layer F.Cu) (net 4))
 (segment (start 193.03 105.23) (end 192.67 105.59) (width 0.2032) (layer F.Cu) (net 4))
 (segment (start 192.67 105.59) (end 192.67 107.23) (width 0.2032) (layer F.Cu) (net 4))
 (segment (start 192.67 107.23) (end 185.54 114.36) (width 0.2032) (layer F.Cu) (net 4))
 (segment (start 185.54 114.36) (end 185.54 116.2) (width 0.2032) (layer F.Cu) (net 4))
 (segment (start 194.22 105.23) (end 194.22 105.37) (width 0.25) (layer F.Cu) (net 4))
 (segment (start 194.22 105.1) (end 194.22 105.23) (width 0.25) (layer F.Cu) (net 4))
 (segment (start 185.54 116.2) (end 186.54 117.2) (width 0.2032) (layer B.Cu) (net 4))
 (segment (start 186.54 117.2) (end 191.3 117.2) (width 0.2032) (layer B.Cu) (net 4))
 (via (at 185.54 116.2) (size 0.6) (layers F.Cu B.Cu) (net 4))
 (segment (start 191.3 119.2) (end 187.54 119.2) (width 0.2032) (layer B.Cu) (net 5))
 (segment (start 187.54 119.2) (end 186.5 118.16) (width 0.2032) (layer B.Cu) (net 5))
 (segment (start 194.18 107.23) (end 193.51 107.23) (width 0.2032) (layer F.Cu) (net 5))
 (segment (start 193.51 107.23) (end 186.5 114.24) (width 0.2032) (layer F.Cu) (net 5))
 (segment (start 186.5 114.24) (end 186.5 118.16) (width 0.2032) (layer F.Cu) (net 5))
 (via (at 186.5 118.16) (size 0.6) (layers F.Cu B.Cu) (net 5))
 (segment (start 194.18 109.1) (end 193.94 109.1) (width 0.2) (layer B.Cu) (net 6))
 (segment (start 194.22 109.1) (end 194.18 109.1) (width 0.2) (layer B.Cu) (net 6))
 (segment (start 194.18 109.23) (end 194.18 109.1) (width 0.2032) (layer B.Cu) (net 6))
 (segment (start 191.3 121.2) (end 188.56 121.2) (width 0.2032) (layer B.Cu) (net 6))
 (segment (start 188.56 121.2) (end 187.37 120.01) (width 0.2032) (layer B.Cu) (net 6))
 (segment (start 194.18 109.23) (end 192.23 109.23) (width 0.2032) (layer F.Cu) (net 6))
 (segment (start 192.23 109.23) (end 187.37 114.09) (width 0.2032) (layer F.Cu) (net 6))
 (segment (start 187.37 114.09) (end 187.37 120.01) (width 0.2032) (layer F.Cu) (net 6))
 (via (at 187.37 120.01) (size 0.6) (layers F.Cu B.Cu) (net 6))
 (segment (start 172.18 111.23) (end 173.012 110.398) (width 0.2032) (layer B.Cu) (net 18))
 (segment (start 173.012 110.398) (end 176.541 110.398) (width 0.2032) (layer B.Cu) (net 18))
 (segment (start 176.541 110.398) (end 178 111.857) (width 0.2032) (layer B.Cu) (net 18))
 (segment (start 178 111.857) (end 178 117) (width 0.2032) (layer B.Cu) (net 18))
 (segment (start 178 117) (end 175.8 119.2) (width 0.2032) (layer B.Cu) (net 18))
 (segment (start 175.8 119.2) (end 175.3 119.2) (width 0.2032) (layer B.Cu) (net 18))
 (segment (start 172.18 121.23) (end 173.6 119.81) (width 0.2032) (layer B.Cu) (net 14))
 (segment (start 173.6 119.81) (end 173.6 118.4) (width 0.2032) (layer B.Cu) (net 14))
 (segment (start 173.6 118.4) (end 174.8 117.2) (width 0.2032) (layer B.Cu) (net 14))
 (segment (start 174.8 117.2) (end 175.3 117.2) (width 0.2032) (layer B.Cu) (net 14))
 (segment (start 194.175 113.1) (end 194.18 113.105) (width 0.2032) (layer B.Cu) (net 8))
 (segment (start 194.18 113.105) (end 194.18 113.23) (width 0.2032) (layer B.Cu) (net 8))
 (segment (start 194.175 113.1) (end 194.13 113.1) (width 0.2) (layer B.Cu) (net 8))
 (segment (start 194.22 113.1) (end 194.175 113.1) (width 0.2) (layer B.Cu) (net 8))
 (segment (start 194.05 121.1) (end 194.18 121.23) (width 0.2032) (layer B.Cu) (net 12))
 (segment (start 194.05 121.1) (end 193.66 121.1) (width 0.2) (layer B.Cu) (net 12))
 (segment (start 194.22 121.1) (end 194.05 121.1) (width 0.2) (layer B.Cu) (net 12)))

